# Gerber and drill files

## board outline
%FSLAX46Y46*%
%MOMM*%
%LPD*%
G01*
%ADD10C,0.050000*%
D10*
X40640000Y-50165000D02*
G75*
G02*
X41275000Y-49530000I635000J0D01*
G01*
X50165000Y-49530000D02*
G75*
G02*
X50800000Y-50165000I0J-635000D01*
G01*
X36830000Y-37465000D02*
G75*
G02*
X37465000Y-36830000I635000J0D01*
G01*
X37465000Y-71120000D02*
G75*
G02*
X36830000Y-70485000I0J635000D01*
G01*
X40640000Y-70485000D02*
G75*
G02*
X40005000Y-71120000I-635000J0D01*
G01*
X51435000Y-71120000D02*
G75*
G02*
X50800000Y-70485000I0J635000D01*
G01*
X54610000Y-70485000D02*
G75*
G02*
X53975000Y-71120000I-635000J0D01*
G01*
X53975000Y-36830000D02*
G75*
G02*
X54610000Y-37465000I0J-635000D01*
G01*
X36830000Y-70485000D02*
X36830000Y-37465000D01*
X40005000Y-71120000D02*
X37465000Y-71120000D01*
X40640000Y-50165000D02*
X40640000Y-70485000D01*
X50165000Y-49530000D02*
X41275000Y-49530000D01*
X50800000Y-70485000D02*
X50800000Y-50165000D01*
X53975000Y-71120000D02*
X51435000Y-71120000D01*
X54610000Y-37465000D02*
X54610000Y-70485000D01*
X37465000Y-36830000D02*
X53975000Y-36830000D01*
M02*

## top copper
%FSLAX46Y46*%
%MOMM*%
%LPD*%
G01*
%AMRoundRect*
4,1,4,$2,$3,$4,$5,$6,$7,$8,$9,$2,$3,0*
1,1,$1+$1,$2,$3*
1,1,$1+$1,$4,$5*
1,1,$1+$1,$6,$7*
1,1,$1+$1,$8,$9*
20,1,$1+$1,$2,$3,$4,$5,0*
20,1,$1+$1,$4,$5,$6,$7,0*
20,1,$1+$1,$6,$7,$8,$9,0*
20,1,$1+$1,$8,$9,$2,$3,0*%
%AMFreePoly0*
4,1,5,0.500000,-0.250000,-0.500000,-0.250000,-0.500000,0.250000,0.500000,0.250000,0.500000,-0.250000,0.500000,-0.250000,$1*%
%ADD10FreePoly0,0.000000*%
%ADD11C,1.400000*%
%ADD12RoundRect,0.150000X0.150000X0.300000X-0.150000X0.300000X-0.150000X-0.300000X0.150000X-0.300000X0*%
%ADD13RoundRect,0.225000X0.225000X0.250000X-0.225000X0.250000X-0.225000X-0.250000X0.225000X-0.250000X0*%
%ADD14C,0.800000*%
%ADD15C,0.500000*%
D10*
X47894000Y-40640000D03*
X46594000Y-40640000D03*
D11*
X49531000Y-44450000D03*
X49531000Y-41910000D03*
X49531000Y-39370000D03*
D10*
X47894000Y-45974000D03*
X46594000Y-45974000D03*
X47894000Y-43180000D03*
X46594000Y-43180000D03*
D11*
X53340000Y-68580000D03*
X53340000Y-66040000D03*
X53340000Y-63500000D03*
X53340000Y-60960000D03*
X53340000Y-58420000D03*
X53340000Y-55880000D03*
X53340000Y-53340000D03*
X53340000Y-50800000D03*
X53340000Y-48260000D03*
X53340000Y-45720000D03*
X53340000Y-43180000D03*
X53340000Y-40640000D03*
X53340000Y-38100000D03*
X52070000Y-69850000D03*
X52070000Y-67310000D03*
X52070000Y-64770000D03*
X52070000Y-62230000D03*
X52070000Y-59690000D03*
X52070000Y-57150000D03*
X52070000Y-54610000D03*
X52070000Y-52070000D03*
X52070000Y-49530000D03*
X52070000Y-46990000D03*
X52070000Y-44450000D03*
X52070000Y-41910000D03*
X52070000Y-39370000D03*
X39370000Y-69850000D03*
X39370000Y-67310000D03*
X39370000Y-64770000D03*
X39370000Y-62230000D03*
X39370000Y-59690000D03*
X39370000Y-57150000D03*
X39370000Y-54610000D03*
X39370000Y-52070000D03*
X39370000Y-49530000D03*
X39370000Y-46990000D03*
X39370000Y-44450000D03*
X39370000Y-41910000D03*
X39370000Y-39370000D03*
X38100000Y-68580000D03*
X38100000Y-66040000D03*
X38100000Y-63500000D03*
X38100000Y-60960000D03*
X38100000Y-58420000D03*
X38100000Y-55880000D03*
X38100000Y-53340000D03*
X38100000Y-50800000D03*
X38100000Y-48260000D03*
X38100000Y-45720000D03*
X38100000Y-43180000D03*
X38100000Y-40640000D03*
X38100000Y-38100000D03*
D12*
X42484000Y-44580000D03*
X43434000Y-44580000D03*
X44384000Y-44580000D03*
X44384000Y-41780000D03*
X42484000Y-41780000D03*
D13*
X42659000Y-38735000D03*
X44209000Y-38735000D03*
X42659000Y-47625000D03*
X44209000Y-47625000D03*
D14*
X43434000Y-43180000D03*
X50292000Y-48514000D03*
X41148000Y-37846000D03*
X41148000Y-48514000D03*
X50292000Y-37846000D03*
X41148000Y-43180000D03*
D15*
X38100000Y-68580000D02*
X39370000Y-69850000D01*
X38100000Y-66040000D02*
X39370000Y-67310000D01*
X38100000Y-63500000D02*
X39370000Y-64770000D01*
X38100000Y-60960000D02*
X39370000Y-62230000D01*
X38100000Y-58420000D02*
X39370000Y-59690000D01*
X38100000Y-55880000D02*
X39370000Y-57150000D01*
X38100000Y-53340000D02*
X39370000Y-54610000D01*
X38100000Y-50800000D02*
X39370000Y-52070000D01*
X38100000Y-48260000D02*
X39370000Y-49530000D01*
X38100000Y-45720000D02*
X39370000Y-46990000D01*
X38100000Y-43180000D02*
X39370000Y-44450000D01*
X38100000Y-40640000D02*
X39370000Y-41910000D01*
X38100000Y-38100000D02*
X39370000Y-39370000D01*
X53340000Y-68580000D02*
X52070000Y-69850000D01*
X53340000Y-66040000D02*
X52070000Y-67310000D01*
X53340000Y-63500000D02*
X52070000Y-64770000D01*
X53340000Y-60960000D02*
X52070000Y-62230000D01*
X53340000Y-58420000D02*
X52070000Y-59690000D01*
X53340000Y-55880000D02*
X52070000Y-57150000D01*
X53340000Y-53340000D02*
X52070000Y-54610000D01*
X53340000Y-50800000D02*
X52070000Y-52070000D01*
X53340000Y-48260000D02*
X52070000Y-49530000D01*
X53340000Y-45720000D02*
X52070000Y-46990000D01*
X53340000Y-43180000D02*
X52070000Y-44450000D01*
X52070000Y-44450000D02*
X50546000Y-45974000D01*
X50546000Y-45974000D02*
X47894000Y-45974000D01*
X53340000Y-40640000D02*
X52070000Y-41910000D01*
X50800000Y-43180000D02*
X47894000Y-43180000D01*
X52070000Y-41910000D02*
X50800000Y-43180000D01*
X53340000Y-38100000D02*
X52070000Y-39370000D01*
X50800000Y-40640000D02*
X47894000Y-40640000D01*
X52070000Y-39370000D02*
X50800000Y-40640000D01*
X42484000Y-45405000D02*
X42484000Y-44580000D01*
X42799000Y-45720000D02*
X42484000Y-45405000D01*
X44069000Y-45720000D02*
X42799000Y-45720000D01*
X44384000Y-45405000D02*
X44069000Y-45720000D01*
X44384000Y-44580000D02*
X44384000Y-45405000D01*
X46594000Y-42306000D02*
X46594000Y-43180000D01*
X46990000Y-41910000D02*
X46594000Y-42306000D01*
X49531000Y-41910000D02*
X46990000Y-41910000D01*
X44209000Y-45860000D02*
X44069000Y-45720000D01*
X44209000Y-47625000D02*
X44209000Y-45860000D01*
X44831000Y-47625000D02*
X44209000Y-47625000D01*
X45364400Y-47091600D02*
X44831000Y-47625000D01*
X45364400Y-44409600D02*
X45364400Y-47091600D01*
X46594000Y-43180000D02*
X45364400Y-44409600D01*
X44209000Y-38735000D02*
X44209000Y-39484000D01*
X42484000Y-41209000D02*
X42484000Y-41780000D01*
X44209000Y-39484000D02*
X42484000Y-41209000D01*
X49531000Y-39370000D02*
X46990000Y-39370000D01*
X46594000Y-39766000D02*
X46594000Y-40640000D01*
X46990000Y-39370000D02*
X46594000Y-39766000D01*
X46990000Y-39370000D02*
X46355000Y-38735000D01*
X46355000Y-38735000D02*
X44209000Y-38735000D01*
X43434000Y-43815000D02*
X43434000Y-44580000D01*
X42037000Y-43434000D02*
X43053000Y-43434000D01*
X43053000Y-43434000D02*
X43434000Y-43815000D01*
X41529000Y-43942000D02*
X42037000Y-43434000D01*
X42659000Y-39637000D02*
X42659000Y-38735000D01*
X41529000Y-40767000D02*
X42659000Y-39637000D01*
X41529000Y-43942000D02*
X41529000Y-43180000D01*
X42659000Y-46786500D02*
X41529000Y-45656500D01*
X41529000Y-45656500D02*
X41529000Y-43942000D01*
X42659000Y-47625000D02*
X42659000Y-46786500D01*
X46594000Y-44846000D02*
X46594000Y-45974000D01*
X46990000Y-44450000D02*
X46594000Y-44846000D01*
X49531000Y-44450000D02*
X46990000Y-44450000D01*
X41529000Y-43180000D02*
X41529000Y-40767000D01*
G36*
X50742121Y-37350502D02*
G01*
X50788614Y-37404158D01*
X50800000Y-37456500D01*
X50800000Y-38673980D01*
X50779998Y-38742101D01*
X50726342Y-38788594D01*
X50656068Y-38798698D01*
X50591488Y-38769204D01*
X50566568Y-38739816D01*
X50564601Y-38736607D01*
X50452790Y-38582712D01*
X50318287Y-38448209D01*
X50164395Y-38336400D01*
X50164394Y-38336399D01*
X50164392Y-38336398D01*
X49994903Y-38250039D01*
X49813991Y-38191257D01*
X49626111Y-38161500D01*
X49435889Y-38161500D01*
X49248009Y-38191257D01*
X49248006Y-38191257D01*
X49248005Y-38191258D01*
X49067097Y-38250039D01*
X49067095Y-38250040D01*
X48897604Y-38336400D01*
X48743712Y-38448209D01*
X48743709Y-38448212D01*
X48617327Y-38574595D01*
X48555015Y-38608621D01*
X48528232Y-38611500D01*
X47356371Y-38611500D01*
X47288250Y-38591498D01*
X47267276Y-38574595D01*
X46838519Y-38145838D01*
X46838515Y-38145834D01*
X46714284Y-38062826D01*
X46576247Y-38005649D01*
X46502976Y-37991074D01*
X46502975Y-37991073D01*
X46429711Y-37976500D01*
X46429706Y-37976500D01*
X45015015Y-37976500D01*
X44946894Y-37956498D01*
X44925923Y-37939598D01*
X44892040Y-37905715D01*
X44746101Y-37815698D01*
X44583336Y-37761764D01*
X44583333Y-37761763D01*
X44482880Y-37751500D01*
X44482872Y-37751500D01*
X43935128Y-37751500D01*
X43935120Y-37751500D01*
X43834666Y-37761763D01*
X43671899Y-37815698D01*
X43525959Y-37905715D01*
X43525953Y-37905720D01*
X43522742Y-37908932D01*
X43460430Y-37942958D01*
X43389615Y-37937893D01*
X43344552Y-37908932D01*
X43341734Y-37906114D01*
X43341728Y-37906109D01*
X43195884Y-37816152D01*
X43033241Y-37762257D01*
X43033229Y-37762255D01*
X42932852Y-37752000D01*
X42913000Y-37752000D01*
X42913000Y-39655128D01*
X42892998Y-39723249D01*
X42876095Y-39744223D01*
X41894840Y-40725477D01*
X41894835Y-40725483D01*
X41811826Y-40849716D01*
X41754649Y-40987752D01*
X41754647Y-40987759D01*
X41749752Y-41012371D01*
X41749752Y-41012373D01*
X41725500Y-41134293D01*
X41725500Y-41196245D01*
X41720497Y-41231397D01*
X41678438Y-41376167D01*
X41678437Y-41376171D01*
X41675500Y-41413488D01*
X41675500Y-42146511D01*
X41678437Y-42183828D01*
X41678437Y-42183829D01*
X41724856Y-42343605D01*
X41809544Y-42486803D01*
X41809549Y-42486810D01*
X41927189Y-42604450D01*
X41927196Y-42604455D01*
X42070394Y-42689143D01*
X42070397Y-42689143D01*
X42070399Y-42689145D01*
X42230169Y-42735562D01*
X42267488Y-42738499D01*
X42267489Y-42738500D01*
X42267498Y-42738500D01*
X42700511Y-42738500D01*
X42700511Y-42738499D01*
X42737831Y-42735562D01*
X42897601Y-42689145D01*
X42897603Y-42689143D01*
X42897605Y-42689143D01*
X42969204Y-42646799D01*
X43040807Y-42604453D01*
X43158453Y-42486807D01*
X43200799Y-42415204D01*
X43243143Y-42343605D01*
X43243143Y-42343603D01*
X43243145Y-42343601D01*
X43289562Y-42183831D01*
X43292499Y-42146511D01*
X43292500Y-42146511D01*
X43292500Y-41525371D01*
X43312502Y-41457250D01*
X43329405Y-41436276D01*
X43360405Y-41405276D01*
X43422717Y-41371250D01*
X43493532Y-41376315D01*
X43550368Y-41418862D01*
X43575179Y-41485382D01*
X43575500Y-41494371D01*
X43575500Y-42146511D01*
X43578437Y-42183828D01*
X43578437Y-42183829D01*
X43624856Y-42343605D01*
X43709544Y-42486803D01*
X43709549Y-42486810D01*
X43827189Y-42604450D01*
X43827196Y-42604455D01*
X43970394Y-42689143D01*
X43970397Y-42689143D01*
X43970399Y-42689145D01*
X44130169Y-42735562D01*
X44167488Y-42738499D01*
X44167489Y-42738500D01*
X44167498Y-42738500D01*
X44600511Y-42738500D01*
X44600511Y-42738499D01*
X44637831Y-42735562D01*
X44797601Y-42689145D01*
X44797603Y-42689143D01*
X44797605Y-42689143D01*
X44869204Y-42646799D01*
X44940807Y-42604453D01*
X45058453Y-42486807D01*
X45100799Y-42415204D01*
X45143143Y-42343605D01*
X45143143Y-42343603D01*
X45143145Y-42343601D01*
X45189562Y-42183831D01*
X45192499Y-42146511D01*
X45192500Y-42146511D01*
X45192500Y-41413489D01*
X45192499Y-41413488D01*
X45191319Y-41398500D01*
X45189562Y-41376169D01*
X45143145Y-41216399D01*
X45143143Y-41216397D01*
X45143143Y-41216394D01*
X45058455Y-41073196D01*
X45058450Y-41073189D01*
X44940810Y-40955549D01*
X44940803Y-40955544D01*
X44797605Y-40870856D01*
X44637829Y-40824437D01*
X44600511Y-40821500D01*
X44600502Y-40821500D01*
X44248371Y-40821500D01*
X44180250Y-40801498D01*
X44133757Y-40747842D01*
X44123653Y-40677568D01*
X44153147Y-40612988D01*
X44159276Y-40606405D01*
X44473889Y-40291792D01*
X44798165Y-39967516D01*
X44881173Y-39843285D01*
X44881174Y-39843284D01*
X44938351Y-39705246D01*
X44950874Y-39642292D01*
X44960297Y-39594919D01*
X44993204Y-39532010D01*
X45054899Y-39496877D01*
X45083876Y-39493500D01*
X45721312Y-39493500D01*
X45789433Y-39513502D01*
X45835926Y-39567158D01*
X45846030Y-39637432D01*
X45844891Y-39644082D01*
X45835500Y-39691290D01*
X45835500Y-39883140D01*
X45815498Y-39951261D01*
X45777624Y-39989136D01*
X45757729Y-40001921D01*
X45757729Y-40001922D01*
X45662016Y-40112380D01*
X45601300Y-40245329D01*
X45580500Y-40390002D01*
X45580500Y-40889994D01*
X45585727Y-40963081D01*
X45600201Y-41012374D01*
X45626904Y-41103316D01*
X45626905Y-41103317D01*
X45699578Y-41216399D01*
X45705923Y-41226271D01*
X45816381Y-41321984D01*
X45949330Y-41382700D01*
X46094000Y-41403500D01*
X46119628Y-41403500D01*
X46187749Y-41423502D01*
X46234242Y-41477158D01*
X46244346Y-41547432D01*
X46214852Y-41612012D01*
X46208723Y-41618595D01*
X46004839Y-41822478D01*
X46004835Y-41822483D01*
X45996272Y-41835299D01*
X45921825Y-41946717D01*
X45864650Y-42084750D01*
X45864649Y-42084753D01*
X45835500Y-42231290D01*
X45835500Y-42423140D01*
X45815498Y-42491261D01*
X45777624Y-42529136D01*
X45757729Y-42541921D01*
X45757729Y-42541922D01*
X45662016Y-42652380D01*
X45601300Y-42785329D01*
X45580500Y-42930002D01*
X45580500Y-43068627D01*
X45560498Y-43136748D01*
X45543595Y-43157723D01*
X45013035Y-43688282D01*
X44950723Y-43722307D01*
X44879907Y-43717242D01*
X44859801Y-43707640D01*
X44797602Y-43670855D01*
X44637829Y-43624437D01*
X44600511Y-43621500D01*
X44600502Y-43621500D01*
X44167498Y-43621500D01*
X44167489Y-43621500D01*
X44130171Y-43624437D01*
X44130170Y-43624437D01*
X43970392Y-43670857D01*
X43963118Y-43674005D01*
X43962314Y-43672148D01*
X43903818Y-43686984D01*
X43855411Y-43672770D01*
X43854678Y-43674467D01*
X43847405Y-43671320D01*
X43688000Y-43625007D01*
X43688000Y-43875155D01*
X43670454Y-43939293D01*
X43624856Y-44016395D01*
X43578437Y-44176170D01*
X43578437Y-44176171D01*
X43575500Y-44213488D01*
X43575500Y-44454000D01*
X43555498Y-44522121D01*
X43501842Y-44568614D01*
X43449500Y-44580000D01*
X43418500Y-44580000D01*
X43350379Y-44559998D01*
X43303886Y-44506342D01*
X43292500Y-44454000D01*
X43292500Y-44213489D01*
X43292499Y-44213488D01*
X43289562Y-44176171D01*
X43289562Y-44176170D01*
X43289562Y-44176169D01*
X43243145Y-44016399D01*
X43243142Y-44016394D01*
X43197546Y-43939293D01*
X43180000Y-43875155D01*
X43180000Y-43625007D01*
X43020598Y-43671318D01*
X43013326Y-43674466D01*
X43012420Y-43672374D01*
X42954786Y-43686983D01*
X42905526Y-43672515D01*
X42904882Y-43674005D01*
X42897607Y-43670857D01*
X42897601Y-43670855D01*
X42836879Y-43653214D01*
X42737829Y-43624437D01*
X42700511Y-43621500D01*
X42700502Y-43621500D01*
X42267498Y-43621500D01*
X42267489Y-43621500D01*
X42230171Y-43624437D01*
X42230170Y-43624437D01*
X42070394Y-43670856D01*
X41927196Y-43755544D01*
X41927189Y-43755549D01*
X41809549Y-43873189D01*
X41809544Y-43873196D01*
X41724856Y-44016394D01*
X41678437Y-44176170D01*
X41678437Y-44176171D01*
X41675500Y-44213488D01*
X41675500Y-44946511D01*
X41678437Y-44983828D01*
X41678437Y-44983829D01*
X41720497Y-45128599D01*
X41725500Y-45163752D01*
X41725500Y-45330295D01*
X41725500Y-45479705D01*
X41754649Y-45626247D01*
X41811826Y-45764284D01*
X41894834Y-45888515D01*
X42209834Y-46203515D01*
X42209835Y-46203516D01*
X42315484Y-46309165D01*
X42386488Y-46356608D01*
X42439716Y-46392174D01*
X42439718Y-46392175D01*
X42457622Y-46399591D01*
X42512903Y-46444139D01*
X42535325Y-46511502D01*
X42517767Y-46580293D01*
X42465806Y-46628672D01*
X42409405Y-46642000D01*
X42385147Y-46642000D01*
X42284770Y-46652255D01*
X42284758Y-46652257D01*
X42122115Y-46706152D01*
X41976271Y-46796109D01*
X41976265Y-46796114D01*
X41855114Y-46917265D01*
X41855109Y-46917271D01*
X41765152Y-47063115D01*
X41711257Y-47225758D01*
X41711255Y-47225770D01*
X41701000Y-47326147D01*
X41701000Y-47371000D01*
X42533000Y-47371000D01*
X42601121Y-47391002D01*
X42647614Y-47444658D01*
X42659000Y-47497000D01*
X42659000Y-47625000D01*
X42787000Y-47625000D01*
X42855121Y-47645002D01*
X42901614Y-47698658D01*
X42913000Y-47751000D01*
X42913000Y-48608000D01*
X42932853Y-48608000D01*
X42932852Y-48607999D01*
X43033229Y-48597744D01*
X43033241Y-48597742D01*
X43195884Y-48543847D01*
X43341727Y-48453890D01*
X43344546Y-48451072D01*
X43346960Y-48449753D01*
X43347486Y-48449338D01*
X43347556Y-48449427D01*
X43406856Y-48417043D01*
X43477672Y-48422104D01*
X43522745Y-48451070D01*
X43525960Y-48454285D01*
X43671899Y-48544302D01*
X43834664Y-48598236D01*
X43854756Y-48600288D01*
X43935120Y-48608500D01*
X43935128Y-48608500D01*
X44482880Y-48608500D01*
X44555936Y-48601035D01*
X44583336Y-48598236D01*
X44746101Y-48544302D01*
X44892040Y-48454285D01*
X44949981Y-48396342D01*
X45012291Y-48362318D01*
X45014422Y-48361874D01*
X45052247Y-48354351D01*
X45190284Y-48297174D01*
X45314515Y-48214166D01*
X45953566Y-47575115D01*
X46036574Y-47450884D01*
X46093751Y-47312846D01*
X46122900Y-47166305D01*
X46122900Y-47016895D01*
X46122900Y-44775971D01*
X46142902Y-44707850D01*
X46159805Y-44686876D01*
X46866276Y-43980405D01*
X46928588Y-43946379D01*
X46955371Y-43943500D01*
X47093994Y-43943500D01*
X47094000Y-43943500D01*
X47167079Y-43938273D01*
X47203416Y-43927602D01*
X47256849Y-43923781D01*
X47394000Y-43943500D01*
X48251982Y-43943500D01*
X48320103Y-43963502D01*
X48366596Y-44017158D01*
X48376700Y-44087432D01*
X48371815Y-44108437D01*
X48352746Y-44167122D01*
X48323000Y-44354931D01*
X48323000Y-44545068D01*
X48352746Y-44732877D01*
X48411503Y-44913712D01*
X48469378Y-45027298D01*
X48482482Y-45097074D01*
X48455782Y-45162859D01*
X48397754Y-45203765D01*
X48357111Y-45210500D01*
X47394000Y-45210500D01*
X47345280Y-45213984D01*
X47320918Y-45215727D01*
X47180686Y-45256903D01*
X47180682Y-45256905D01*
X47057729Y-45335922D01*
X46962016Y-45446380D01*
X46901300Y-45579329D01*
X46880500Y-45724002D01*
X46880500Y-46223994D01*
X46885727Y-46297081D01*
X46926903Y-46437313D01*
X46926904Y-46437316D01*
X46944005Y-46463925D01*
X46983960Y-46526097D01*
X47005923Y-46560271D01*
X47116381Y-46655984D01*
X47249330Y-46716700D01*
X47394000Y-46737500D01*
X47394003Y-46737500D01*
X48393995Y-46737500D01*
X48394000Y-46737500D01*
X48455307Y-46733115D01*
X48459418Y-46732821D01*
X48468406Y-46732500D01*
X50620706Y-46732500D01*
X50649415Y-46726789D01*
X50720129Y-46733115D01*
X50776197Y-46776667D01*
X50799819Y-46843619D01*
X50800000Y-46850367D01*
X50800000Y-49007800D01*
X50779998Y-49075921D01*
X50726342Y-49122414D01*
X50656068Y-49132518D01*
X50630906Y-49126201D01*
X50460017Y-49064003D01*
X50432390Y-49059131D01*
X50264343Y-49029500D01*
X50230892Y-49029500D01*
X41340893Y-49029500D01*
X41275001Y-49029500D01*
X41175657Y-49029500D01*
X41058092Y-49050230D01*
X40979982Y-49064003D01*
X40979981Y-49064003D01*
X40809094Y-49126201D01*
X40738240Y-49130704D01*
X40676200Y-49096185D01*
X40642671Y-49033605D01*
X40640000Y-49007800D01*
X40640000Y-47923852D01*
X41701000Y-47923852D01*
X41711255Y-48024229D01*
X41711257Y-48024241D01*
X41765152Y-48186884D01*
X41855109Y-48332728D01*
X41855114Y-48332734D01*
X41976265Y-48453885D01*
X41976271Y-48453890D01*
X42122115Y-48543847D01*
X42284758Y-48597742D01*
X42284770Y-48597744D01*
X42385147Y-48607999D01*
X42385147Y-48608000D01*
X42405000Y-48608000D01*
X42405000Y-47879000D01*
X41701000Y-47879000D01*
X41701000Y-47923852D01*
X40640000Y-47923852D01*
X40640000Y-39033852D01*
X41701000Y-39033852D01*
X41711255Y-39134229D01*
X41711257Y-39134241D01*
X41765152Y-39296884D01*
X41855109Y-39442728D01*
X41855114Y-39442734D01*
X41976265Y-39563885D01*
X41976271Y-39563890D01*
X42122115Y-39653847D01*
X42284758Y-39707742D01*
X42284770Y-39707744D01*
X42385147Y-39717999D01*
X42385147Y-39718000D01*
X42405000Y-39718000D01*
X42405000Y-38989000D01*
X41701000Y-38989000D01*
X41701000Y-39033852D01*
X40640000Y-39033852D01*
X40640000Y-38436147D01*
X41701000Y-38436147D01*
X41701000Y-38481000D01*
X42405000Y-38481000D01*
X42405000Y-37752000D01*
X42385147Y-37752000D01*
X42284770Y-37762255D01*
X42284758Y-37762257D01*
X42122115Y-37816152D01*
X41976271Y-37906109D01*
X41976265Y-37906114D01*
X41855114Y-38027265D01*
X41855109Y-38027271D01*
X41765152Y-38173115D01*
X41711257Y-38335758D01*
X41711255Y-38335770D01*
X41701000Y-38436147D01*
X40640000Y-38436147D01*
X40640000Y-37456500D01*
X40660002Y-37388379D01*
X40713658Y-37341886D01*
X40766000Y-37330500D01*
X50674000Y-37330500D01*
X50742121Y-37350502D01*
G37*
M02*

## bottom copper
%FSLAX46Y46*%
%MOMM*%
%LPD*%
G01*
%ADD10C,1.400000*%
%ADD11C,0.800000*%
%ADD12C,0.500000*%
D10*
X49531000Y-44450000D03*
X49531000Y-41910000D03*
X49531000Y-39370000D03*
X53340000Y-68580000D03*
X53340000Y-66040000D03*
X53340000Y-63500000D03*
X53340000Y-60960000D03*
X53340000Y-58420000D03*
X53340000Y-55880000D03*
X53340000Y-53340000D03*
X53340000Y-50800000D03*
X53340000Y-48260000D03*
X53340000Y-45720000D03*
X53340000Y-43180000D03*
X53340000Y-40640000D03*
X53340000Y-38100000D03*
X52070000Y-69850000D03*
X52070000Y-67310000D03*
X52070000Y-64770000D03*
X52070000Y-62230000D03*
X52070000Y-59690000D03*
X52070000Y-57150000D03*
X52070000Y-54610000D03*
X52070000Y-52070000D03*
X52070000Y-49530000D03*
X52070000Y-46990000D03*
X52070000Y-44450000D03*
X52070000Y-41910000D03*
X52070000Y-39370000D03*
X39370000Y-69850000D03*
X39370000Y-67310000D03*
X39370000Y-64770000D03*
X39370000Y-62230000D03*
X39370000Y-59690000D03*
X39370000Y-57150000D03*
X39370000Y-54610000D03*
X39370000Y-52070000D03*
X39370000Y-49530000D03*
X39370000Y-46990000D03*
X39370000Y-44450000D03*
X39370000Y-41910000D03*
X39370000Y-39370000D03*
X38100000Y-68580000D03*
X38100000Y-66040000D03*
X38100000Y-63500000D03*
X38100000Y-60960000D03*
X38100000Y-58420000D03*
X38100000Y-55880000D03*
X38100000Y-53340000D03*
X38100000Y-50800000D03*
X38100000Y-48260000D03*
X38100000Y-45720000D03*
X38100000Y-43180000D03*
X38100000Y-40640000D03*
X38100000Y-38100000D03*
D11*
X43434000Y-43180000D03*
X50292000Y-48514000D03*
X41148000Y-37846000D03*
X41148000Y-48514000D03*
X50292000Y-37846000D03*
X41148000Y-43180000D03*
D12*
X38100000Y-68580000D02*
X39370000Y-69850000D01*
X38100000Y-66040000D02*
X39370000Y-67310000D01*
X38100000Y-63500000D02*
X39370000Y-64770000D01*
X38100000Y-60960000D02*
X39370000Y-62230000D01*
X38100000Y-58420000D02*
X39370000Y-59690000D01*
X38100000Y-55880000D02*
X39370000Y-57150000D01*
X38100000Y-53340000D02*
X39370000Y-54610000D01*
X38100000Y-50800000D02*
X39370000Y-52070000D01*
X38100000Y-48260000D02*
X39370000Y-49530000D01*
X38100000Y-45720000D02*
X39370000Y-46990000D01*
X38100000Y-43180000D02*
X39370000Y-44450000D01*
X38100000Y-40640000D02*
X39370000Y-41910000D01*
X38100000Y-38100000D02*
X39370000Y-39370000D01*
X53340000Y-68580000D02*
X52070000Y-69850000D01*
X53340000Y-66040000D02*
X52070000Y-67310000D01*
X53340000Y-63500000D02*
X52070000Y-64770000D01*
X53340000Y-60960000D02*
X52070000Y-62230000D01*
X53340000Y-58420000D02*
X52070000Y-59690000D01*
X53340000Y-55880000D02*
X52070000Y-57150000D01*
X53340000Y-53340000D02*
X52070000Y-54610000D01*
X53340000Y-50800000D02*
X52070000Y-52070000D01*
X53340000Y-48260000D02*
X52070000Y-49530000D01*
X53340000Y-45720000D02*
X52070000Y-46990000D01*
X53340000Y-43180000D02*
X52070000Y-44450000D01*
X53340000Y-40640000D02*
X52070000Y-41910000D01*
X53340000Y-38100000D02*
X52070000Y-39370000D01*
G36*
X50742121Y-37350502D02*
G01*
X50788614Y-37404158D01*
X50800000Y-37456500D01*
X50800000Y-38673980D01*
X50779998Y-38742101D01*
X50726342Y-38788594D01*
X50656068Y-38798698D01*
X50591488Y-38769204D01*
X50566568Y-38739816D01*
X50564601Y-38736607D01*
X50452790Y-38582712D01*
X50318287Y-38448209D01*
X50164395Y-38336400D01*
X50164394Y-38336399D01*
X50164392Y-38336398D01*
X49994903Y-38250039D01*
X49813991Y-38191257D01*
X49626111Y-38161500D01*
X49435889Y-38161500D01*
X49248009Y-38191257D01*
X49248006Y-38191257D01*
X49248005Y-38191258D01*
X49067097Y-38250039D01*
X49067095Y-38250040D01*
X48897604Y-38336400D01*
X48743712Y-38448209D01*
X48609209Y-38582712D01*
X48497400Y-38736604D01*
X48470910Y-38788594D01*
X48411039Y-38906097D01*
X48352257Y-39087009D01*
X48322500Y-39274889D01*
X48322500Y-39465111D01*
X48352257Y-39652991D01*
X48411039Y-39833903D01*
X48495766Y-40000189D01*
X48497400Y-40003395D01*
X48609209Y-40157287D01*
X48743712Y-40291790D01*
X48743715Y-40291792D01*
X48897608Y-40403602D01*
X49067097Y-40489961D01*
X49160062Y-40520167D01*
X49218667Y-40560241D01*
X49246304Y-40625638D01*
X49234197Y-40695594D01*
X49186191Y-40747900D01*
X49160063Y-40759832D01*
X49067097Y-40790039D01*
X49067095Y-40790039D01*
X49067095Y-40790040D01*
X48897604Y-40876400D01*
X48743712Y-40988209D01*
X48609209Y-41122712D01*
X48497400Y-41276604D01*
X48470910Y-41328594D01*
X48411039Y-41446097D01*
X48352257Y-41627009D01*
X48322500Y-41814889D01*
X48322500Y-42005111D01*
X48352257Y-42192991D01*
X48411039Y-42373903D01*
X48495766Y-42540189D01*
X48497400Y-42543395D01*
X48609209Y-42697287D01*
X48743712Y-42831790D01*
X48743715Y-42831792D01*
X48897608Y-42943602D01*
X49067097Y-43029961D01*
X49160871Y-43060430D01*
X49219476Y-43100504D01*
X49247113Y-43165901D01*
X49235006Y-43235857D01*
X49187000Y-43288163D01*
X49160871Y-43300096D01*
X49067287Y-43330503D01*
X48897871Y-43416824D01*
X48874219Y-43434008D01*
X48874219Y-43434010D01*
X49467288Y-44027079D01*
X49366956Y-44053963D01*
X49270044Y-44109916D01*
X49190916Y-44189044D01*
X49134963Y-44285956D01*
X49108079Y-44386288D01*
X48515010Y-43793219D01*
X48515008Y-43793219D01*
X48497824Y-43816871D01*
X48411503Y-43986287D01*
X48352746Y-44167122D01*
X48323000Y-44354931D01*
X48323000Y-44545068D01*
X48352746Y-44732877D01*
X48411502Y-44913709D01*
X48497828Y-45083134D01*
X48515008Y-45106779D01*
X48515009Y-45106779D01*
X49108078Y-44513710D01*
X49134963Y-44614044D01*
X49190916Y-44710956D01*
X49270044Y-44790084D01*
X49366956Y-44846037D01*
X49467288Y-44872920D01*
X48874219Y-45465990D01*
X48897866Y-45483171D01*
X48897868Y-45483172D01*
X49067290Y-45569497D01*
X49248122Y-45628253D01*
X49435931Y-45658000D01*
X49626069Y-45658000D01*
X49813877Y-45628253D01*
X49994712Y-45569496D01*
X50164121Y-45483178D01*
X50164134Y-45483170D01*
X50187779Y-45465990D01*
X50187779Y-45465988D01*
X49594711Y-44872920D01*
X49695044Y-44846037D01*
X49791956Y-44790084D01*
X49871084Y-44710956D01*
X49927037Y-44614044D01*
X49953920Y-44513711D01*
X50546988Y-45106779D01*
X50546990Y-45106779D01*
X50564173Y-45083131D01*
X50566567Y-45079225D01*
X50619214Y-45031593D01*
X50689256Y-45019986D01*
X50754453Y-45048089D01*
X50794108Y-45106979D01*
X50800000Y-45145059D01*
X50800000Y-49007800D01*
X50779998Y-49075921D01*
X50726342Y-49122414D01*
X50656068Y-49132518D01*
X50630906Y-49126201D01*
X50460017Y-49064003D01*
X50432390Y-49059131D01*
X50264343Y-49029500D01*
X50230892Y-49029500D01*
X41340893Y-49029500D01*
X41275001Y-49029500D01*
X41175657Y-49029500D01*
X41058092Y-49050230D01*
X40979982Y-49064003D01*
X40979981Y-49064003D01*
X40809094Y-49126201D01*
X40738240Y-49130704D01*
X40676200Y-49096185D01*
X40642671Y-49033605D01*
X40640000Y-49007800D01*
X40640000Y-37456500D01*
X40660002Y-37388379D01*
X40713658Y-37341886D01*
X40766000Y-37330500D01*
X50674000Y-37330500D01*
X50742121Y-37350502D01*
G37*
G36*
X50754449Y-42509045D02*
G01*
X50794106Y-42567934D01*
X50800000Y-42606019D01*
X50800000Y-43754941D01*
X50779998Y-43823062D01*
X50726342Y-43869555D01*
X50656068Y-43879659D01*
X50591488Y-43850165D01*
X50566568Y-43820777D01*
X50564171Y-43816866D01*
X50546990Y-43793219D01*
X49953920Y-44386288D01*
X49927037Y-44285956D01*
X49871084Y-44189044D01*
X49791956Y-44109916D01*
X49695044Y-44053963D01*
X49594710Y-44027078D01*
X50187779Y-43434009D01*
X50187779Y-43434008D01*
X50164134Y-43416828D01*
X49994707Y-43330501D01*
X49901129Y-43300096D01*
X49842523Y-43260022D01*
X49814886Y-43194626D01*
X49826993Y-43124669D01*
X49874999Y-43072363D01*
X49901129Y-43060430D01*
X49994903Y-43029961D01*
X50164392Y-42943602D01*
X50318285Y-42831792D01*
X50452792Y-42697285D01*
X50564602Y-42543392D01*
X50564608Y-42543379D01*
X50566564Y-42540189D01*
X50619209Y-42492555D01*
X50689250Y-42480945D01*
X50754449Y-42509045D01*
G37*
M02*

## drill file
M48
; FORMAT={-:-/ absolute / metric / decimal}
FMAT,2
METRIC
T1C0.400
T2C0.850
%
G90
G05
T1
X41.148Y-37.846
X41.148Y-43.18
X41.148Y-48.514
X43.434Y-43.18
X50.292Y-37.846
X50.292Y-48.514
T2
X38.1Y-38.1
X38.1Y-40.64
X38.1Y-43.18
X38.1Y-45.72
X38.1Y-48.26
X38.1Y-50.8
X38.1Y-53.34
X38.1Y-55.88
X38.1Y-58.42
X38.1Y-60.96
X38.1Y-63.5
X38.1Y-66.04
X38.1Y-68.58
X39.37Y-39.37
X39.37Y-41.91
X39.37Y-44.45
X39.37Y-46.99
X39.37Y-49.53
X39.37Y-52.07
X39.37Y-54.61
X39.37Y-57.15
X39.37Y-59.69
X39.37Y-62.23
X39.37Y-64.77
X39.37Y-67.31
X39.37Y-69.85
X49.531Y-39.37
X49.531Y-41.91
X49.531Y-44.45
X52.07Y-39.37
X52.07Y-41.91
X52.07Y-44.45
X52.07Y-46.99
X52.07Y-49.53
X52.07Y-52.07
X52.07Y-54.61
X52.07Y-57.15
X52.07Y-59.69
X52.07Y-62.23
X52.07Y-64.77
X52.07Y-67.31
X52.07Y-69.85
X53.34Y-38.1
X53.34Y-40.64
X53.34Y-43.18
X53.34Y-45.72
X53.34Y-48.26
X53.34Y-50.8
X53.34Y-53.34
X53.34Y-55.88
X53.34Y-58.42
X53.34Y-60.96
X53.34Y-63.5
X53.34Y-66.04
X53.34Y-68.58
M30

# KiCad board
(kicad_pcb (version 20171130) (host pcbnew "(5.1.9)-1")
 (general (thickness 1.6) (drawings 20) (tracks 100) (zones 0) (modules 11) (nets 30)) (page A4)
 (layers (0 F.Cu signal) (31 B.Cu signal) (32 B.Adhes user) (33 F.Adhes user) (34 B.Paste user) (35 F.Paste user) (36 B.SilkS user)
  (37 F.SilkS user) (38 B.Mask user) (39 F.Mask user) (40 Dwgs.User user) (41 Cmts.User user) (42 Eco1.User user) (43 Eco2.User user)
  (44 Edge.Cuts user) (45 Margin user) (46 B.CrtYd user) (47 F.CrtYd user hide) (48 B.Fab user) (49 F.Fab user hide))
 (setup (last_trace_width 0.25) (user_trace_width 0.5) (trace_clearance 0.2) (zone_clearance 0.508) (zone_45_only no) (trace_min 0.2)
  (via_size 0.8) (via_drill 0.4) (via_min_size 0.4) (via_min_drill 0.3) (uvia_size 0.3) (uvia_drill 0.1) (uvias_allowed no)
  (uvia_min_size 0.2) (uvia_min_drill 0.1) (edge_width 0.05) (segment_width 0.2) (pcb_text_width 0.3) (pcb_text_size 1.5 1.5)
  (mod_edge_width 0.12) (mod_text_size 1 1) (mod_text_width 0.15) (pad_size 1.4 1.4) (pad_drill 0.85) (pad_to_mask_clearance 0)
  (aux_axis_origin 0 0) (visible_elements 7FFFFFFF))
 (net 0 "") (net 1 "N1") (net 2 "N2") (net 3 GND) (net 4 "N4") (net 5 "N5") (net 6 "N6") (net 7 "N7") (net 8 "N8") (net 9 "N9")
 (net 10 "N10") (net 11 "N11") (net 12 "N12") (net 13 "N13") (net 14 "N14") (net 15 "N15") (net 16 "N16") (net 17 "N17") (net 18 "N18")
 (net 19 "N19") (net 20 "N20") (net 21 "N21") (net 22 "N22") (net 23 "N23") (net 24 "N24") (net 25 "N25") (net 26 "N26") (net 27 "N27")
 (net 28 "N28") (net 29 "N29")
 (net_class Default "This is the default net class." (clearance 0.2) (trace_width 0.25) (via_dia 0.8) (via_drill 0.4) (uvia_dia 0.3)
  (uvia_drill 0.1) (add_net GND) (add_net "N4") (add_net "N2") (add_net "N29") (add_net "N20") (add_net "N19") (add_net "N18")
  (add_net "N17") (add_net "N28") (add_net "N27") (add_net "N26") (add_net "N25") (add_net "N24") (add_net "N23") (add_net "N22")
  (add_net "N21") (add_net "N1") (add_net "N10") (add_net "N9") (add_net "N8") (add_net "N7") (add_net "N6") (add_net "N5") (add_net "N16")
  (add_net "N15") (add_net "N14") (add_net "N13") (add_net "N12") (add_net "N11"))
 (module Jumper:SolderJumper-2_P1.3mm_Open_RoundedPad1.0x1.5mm (layer F.Cu) (at 47.244 40.64)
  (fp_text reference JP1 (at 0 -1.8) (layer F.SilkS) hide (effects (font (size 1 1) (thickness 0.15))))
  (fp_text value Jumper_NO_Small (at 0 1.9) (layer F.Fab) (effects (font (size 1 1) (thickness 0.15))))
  (pad 2 smd custom (at 0.65 0) (size 1 0.5) (layers F.Cu F.Mask) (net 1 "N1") (zone_connect 2) (options (clearance outline) (anchor rect))
   (primitives))
  (pad 1 smd custom (at -0.65 0) (size 1 0.5) (layers F.Cu F.Mask) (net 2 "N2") (zone_connect 2) (options (clearance outline) (anchor rect))
   (primitives)))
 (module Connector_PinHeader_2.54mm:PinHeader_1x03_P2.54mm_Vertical (layer F.Cu) (at 49.531 39.37)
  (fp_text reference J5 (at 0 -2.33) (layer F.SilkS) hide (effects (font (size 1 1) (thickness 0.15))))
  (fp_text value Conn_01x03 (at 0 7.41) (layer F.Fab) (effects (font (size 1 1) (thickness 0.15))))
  (pad 3 thru_hole circle (at 0 5.08) (size 1.4 1.4) (drill 0.85) (layers *.Cu *.Mask) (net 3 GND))
  (pad 2 thru_hole circle (at 0 2.54) (size 1.4 1.4) (drill 0.85) (layers *.Cu *.Mask) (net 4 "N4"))
  (pad 1 thru_hole circle (at 0 0) (size 1.4 1.4) (drill 0.85) (layers *.Cu *.Mask) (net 2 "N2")))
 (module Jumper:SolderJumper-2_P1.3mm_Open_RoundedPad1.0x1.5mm (layer F.Cu) (at 47.244 45.974)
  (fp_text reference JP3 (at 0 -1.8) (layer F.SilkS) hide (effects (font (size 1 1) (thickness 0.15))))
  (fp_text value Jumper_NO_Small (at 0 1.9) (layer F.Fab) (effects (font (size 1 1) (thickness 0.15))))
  (pad 2 smd custom (at 0.65 0) (size 1 0.5) (layers F.Cu F.Mask) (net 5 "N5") (zone_connect 2) (options (clearance outline) (anchor rect))
   (primitives))
  (pad 1 smd custom (at -0.65 0) (size 1 0.5) (layers F.Cu F.Mask) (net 3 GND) (zone_connect 2) (options (clearance outline) (anchor rect))
   (primitives)))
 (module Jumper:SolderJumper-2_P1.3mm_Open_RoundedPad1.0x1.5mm (layer F.Cu) (at 47.244 43.18)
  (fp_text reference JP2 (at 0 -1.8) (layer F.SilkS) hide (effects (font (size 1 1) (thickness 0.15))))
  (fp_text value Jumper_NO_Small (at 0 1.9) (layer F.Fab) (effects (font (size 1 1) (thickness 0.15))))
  (pad 2 smd custom (at 0.65 0) (size 1 0.5) (layers F.Cu F.Mask) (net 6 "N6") (zone_connect 2) (options (clearance outline) (anchor rect))
   (primitives))
  (pad 1 smd custom (at -0.65 0) (size 1 0.5) (layers F.Cu F.Mask) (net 4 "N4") (zone_connect 2) (options (clearance outline) (anchor rect))
   (primitives)))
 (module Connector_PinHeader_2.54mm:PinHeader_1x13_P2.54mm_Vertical (layer F.Cu) (at 53.34 38.1)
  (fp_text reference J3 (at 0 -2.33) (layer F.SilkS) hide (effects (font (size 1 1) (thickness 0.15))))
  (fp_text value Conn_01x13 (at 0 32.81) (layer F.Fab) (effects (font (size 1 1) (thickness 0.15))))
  (pad 13 thru_hole circle (at 0 30.48) (size 1.4 1.4) (drill 0.85) (layers *.Cu *.Mask) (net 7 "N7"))
  (pad 12 thru_hole circle (at 0 27.94) (size 1.4 1.4) (drill 0.85) (layers *.Cu *.Mask) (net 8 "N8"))
  (pad 11 thru_hole circle (at 0 25.4) (size 1.4 1.4) (drill 0.85) (layers *.Cu *.Mask) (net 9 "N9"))
  (pad 10 thru_hole circle (at 0 22.86) (size 1.4 1.4) (drill 0.85) (layers *.Cu *.Mask) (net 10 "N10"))
  (pad 9 thru_hole circle (at 0 20.32) (size 1.4 1.4) (drill 0.85) (layers *.Cu *.Mask) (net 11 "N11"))
  (pad 8 thru_hole circle (at 0 17.78) (size 1.4 1.4) (drill 0.85) (layers *.Cu *.Mask) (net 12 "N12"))
  (pad 7 thru_hole circle (at 0 15.24) (size 1.4 1.4) (drill 0.85) (layers *.Cu *.Mask) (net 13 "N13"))
  (pad 6 thru_hole circle (at 0 12.7) (size 1.4 1.4) (drill 0.85) (layers *.Cu *.Mask) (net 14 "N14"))
  (pad 5 thru_hole circle (at 0 10.16) (size 1.4 1.4) (drill 0.85) (layers *.Cu *.Mask) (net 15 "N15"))
  (pad 4 thru_hole circle (at 0 7.62) (size 1.4 1.4) (drill 0.85) (layers *.Cu *.Mask) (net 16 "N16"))
  (pad 3 thru_hole circle (at 0 5.08) (size 1.4 1.4) (drill 0.85) (layers *.Cu *.Mask) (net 5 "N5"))
  (pad 2 thru_hole circle (at 0 2.54) (size 1.4 1.4) (drill 0.85) (layers *.Cu *.Mask) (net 6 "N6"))
  (pad 1 thru_hole circle (at 0 0) (size 1.4 1.4) (drill 0.85) (layers *.Cu *.Mask) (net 1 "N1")))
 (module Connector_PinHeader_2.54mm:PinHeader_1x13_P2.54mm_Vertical (layer F.Cu) (at 52.07 39.37)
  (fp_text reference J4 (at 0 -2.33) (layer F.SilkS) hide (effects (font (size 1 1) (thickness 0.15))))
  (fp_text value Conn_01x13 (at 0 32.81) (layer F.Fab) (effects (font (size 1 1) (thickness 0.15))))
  (pad 13 thru_hole circle (at 0 30.48) (size 1.4 1.4) (drill 0.85) (layers *.Cu *.Mask) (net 7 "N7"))
  (pad 12 thru_hole circle (at 0 27.94) (size 1.4 1.4) (drill 0.85) (layers *.Cu *.Mask) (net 8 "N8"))
  (pad 11 thru_hole circle (at 0 25.4) (size 1.4 1.4) (drill 0.85) (layers *.Cu *.Mask) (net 9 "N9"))
  (pad 10 thru_hole circle (at 0 22.86) (size 1.4 1.4) (drill 0.85) (layers *.Cu *.Mask) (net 10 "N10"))
  (pad 9 thru_hole circle (at 0 20.32) (size 1.4 1.4) (drill 0.85) (layers *.Cu *.Mask) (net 11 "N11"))
  (pad 8 thru_hole circle (at 0 17.78) (size 1.4 1.4) (drill 0.85) (layers *.Cu *.Mask) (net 12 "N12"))
  (pad 7 thru_hole circle (at 0 15.24) (size 1.4 1.4) (drill 0.85) (layers *.Cu *.Mask) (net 13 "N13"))
  (pad 6 thru_hole circle (at 0 12.7) (size 1.4 1.4) (drill 0.85) (layers *.Cu *.Mask) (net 14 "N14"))
  (pad 5 thru_hole circle (at 0 10.16) (size 1.4 1.4) (drill 0.85) (layers *.Cu *.Mask) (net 15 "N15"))
  (pad 4 thru_hole circle (at 0 7.62) (size 1.4 1.4) (drill 0.85) (layers *.Cu *.Mask) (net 16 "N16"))
  (pad 3 thru_hole circle (at 0 5.08) (size 1.4 1.4) (drill 0.85) (layers *.Cu *.Mask) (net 5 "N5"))
  (pad 2 thru_hole circle (at 0 2.54) (size 1.4 1.4) (drill 0.85) (layers *.Cu *.Mask) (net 6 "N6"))
  (pad 1 thru_hole circle (at 0 0) (size 1.4 1.4) (drill 0.85) (layers *.Cu *.Mask) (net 1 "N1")))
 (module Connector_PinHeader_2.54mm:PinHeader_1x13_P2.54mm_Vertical (layer F.Cu) (at 39.37 39.37)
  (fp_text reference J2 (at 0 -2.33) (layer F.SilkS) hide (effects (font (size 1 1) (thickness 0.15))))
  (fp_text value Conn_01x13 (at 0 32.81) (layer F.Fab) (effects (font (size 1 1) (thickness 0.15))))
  (pad 13 thru_hole circle (at 0 30.48) (size 1.4 1.4) (drill 0.85) (layers *.Cu *.Mask) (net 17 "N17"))
  (pad 12 thru_hole circle (at 0 27.94) (size 1.4 1.4) (drill 0.85) (layers *.Cu *.Mask) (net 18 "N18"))
  (pad 11 thru_hole circle (at 0 25.4) (size 1.4 1.4) (drill 0.85) (layers *.Cu *.Mask) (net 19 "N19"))
  (pad 10 thru_hole circle (at 0 22.86) (size 1.4 1.4) (drill 0.85) (layers *.Cu *.Mask) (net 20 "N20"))
  (pad 9 thru_hole circle (at 0 20.32) (size 1.4 1.4) (drill 0.85) (layers *.Cu *.Mask) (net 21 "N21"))
  (pad 8 thru_hole circle (at 0 17.78) (size 1.4 1.4) (drill 0.85) (layers *.Cu *.Mask) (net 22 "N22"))
  (pad 7 thru_hole circle (at 0 15.24) (size 1.4 1.4) (drill 0.85) (layers *.Cu *.Mask) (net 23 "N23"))
  (pad 6 thru_hole circle (at 0 12.7) (size 1.4 1.4) (drill 0.85) (layers *.Cu *.Mask) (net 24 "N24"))
  (pad 5 thru_hole circle (at 0 10.16) (size 1.4 1.4) (drill 0.85) (layers *.Cu *.Mask) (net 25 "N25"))
  (pad 4 thru_hole circle (at 0 7.62) (size 1.4 1.4) (drill 0.85) (layers *.Cu *.Mask) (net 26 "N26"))
  (pad 3 thru_hole circle (at 0 5.08) (size 1.4 1.4) (drill 0.85) (layers *.Cu *.Mask) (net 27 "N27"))
  (pad 2 thru_hole circle (at 0 2.54) (size 1.4 1.4) (drill 0.85) (layers *.Cu *.Mask) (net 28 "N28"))
  (pad 1 thru_hole circle (at 0 0) (size 1.4 1.4) (drill 0.85) (layers *.Cu *.Mask) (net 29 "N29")))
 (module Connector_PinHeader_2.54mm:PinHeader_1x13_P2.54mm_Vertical (layer F.Cu) (at 38.1 38.1)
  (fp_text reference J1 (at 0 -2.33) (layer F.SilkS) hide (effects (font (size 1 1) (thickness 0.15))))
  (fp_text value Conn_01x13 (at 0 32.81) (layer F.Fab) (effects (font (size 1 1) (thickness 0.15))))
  (pad 13 thru_hole circle (at 0 30.48) (size 1.4 1.4) (drill 0.85) (layers *.Cu *.Mask) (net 17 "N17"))
  (pad 12 thru_hole circle (at 0 27.94) (size 1.4 1.4) (drill 0.85) (layers *.Cu *.Mask) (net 18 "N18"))
  (pad 11 thru_hole circle (at 0 25.4) (size 1.4 1.4) (drill 0.85) (layers *.Cu *.Mask) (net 19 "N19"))
  (pad 10 thru_hole circle (at 0 22.86) (size 1.4 1.4) (drill 0.85) (layers *.Cu *.Mask) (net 20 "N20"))
  (pad 9 thru_hole circle (at 0 20.32) (size 1.4 1.4) (drill 0.85) (layers *.Cu *.Mask) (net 21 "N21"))
  (pad 8 thru_hole circle (at 0 17.78) (size 1.4 1.4) (drill 0.85) (layers *.Cu *.Mask) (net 22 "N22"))
  (pad 7 thru_hole circle (at 0 15.24) (size 1.4 1.4) (drill 0.85) (layers *.Cu *.Mask) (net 23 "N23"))
  (pad 6 thru_hole circle (at 0 12.7) (size 1.4 1.4) (drill 0.85) (layers *.Cu *.Mask) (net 24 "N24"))
  (pad 5 thru_hole circle (at 0 10.16) (size 1.4 1.4) (drill 0.85) (layers *.Cu *.Mask) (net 25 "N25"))
  (pad 4 thru_hole circle (at 0 7.62) (size 1.4 1.4) (drill 0.85) (layers *.Cu *.Mask) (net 26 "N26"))
  (pad 3 thru_hole circle (at 0 5.08) (size 1.4 1.4) (drill 0.85) (layers *.Cu *.Mask) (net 27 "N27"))
  (pad 2 thru_hole circle (at 0 2.54) (size 1.4 1.4) (drill 0.85) (layers *.Cu *.Mask) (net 28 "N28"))
  (pad 1 thru_hole circle (at 0 0) (size 1.4 1.4) (drill 0.85) (layers *.Cu *.Mask) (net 29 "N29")))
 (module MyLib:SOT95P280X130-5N (layer F.Cu) (at 43.434 43.18 90)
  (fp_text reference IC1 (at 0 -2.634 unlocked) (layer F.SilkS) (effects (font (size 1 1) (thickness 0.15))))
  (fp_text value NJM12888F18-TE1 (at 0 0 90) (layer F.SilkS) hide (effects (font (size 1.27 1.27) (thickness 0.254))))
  (pad 1 smd roundrect (at -1.4 -0.95 180) (size 0.6 0.9) (layers F.Cu F.Paste F.Mask) (roundrect_rratio 0.25) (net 4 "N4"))
  (pad 2 smd roundrect (at -1.4 0 180) (size 0.6 0.9) (layers F.Cu F.Paste F.Mask) (roundrect_rratio 0.25) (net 3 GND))
  (pad 3 smd roundrect (at -1.4 0.95 180) (size 0.6 0.9) (layers F.Cu F.Paste F.Mask) (roundrect_rratio 0.25) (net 4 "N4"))
  (pad 4 smd roundrect (at 1.4 0.95 180) (size 0.6 0.9) (layers F.Cu F.Paste F.Mask) (roundrect_rratio 0.25))
  (pad 5 smd roundrect (at 1.4 -0.95 180) (size 0.6 0.9) (layers F.Cu F.Paste F.Mask) (roundrect_rratio 0.25) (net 2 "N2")))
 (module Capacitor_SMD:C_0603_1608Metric (layer F.Cu) (at 43.434 38.735 180)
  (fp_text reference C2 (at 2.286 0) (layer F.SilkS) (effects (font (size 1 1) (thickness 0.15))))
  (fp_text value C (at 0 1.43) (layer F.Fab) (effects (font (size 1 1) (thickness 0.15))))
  (pad 2 smd roundrect (at 0.775 0 180) (size 0.9 0.95) (layers F.Cu F.Paste F.Mask) (roundrect_rratio 0.25) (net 3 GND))
  (pad 1 smd roundrect (at -0.775 0 180) (size 0.9 0.95) (layers F.Cu F.Paste F.Mask) (roundrect_rratio 0.25) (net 2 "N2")))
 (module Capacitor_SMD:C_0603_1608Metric (layer F.Cu) (at 43.434 47.625 180)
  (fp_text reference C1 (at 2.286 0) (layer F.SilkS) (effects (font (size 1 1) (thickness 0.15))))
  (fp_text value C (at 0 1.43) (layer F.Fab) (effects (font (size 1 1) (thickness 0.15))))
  (pad 2 smd roundrect (at 0.775 0 180) (size 0.9 0.95) (layers F.Cu F.Paste F.Mask) (roundrect_rratio 0.25) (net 3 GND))
  (pad 1 smd roundrect (at -0.775 0 180) (size 0.9 0.95) (layers F.Cu F.Paste F.Mask) (roundrect_rratio 0.25) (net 4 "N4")))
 (gr_arc (start 41.275 50.165) (end 41.275 49.53) (angle -90) (layer Edge.Cuts) (width 0.05))
 (gr_arc (start 50.165 50.165) (end 50.8 50.165) (angle -90) (layer Edge.Cuts) (width 0.05))
 (gr_arc (start 37.465 37.465) (end 37.465 36.83) (angle -90) (layer Edge.Cuts) (width 0.05))
 (gr_arc (start 37.465 70.485) (end 36.83 70.485) (angle -90) (layer Edge.Cuts) (width 0.05))
 (gr_arc (start 40.005 70.485) (end 40.005 71.12) (angle -90) (layer Edge.Cuts) (width 0.05))
 (gr_arc (start 51.435 70.485) (end 50.8 70.485) (angle -90) (layer Edge.Cuts) (width 0.05))
 (gr_arc (start 53.975 70.485) (end 53.975 71.12) (angle -90) (layer Edge.Cuts) (width 0.05))
 (gr_arc (start 53.975 37.465) (end 54.61 37.465) (angle -90) (layer Edge.Cuts) (width 0.05))
 (gr_line (start 36.83 70.485) (end 36.83 37.465) (layer Edge.Cuts) (width 0.05))
 (gr_line (start 40.005 71.12) (end 37.465 71.12) (layer Edge.Cuts) (width 0.05))
 (gr_line (start 40.64 50.165) (end 40.64 70.485) (layer Edge.Cuts) (width 0.05))
 (gr_line (start 50.165 49.53) (end 41.275 49.53) (layer Edge.Cuts) (width 0.05))
 (gr_line (start 50.8 70.485) (end 50.8 50.165) (layer Edge.Cuts) (width 0.05))
 (gr_line (start 53.975 71.12) (end 51.435 71.12) (layer Edge.Cuts) (width 0.05))
 (gr_line (start 54.61 37.465) (end 54.61 70.485) (layer Edge.Cuts) (width 0.05))
 (gr_line (start 37.465 36.83) (end 53.975 36.83) (layer Edge.Cuts) (width 0.05))
 (segment (start 38.1 68.58) (end 39.37 69.85) (width 0.5) (layer B.Cu) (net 17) (status 30))
 (segment (start 38.1 68.58) (end 39.37 69.85) (width 0.5) (layer F.Cu) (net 17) (status 30))
 (segment (start 38.1 66.04) (end 39.37 67.31) (width 0.5) (layer B.Cu) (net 18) (status 30))
 (segment (start 38.1 66.04) (end 39.37 67.31) (width 0.5) (layer F.Cu) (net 18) (status 30))
 (segment (start 38.1 63.5) (end 39.37 64.77) (width 0.5) (layer B.Cu) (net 19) (status 30))
 (segment (start 38.1 63.5) (end 39.37 64.77) (width 0.5) (layer F.Cu) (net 19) (status 30))
 (segment (start 38.1 60.96) (end 39.37 62.23) (width 0.5) (layer B.Cu) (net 20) (status 30))
 (segment (start 38.1 60.96) (end 39.37 62.23) (width 0.5) (layer F.Cu) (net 20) (status 30))
 (segment (start 38.1 58.42) (end 39.37 59.69) (width 0.5) (layer B.Cu) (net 21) (status 30))
 (segment (start 38.1 58.42) (end 39.37 59.69) (width 0.5) (layer F.Cu) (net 21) (status 30))
 (segment (start 38.1 55.88) (end 39.37 57.15) (width 0.5) (layer B.Cu) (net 22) (status 30))
 (segment (start 38.1 55.88) (end 39.37 57.15) (width 0.5) (layer F.Cu) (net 22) (status 30))
 (segment (start 38.1 53.34) (end 39.37 54.61) (width 0.5) (layer B.Cu) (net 23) (status 30))
 (segment (start 38.1 53.34) (end 39.37 54.61) (width 0.5) (layer F.Cu) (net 23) (status 30))
 (segment (start 38.1 50.8) (end 39.37 52.07) (width 0.5) (layer B.Cu) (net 24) (status 30))
 (segment (start 38.1 50.8) (end 39.37 52.07) (width 0.5) (layer F.Cu) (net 24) (status 30))
 (segment (start 38.1 48.26) (end 39.37 49.53) (width 0.5) (layer B.Cu) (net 25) (status 30))
 (segment (start 38.1 48.26) (end 39.37 49.53) (width 0.5) (layer F.Cu) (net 25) (status 30))
 (segment (start 38.1 45.72) (end 39.37 46.99) (width 0.5) (layer B.Cu) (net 26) (status 30))
 (segment (start 38.1 45.72) (end 39.37 46.99) (width 0.5) (layer F.Cu) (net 26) (status 30))
 (segment (start 38.1 43.18) (end 39.37 44.45) (width 0.5) (layer B.Cu) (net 27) (status 30))
 (segment (start 38.1 43.18) (end 39.37 44.45) (width 0.5) (layer F.Cu) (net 27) (status 30))
 (segment (start 38.1 40.64) (end 39.37 41.91) (width 0.5) (layer B.Cu) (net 28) (status 30))
 (segment (start 38.1 40.64) (end 39.37 41.91) (width 0.5) (layer F.Cu) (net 28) (status 30))
 (segment (start 38.1 38.1) (end 39.37 39.37) (width 0.5) (layer B.Cu) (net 29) (status 30))
 (segment (start 38.1 38.1) (end 39.37 39.37) (width 0.5) (layer F.Cu) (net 29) (status 30))
 (segment (start 53.34 68.58) (end 52.07 69.85) (width 0.5) (layer B.Cu) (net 7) (status 30))
 (segment (start 53.34 68.58) (end 52.07 69.85) (width 0.5) (layer F.Cu) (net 7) (status 30))
 (segment (start 53.34 66.04) (end 52.07 67.31) (width 0.5) (layer B.Cu) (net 8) (status 30))
 (segment (start 53.34 66.04) (end 52.07 67.31) (width 0.5) (layer F.Cu) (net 8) (status 30))
 (segment (start 53.34 63.5) (end 52.07 64.77) (width 0.5) (layer B.Cu) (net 9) (status 30))
 (segment (start 53.34 63.5) (end 52.07 64.77) (width 0.5) (layer F.Cu) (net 9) (status 30))
 (segment (start 53.34 60.96) (end 52.07 62.23) (width 0.5) (layer B.Cu) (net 10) (status 30))
 (segment (start 53.34 60.96) (end 52.07 62.23) (width 0.5) (layer F.Cu) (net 10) (status 30))
 (segment (start 53.34 58.42) (end 52.07 59.69) (width 0.5) (layer B.Cu) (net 11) (status 30))
 (segment (start 53.34 58.42) (end 52.07 59.69) (width 0.5) (layer F.Cu) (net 11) (status 30))
 (segment (start 53.34 55.88) (end 52.07 57.15) (width 0.5) (layer B.Cu) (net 12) (status 30))
 (segment (start 53.34 55.88) (end 52.07 57.15) (width 0.5) (layer F.Cu) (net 12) (status 30))
 (segment (start 53.34 53.34) (end 52.07 54.61) (width 0.5) (layer B.Cu) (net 13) (status 30))
 (segment (start 53.34 53.34) (end 52.07 54.61) (width 0.5) (layer F.Cu) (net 13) (status 30))
 (segment (start 53.34 50.8) (end 52.07 52.07) (width 0.5) (layer B.Cu) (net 14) (status 30))
 (segment (start 53.34 50.8) (end 52.07 52.07) (width 0.5) (layer F.Cu) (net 14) (status 30))
 (segment (start 53.34 48.26) (end 52.07 49.53) (width 0.5) (layer B.Cu) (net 15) (status 30))
 (segment (start 53.34 48.26) (end 52.07 49.53) (width 0.5) (layer F.Cu) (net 15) (status 30))
 (segment (start 53.34 45.72) (end 52.07 46.99) (width 0.5) (layer B.Cu) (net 16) (status 30))
 (segment (start 53.34 45.72) (end 52.07 46.99) (width 0.5) (layer F.Cu) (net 16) (status 30))
 (segment (start 53.34 43.18) (end 52.07 44.45) (width 0.5) (layer B.Cu) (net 5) (status 30))
 (segment (start 53.34 43.18) (end 52.07 44.45) (width 0.5) (layer F.Cu) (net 5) (status 30))
 (segment (start 52.07 44.45) (end 50.546 45.974) (width 0.5) (layer F.Cu) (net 5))
 (segment (start 50.546 45.974) (end 47.894 45.974) (width 0.5) (layer F.Cu) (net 5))
 (segment (start 53.34 40.64) (end 52.07 41.91) (width 0.5) (layer B.Cu) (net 6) (status 30))
 (segment (start 53.34 40.64) (end 52.07 41.91) (width 0.5) (layer F.Cu) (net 6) (status 30))
 (segment (start 50.8 43.18) (end 47.894 43.18) (width 0.5) (layer F.Cu) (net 6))
 (segment (start 52.07 41.91) (end 50.8 43.18) (width 0.5) (layer F.Cu) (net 6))
 (segment (start 53.34 38.1) (end 52.07 39.37) (width 0.5) (layer B.Cu) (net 1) (status 30))
 (segment (start 53.34 38.1) (end 52.07 39.37) (width 0.5) (layer F.Cu) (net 1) (status 30))
 (segment (start 50.8 40.64) (end 47.894 40.64) (width 0.5) (layer F.Cu) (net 1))
 (segment (start 52.07 39.37) (end 50.8 40.64) (width 0.5) (layer F.Cu) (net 1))
 (segment (start 42.484 45.405) (end 42.484 44.58) (width 0.5) (layer F.Cu) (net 4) (status 20))
 (segment (start 42.799 45.72) (end 42.484 45.405) (width 0.5) (layer F.Cu) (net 4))
 (segment (start 44.069 45.72) (end 42.799 45.72) (width 0.5) (layer F.Cu) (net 4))
 (segment (start 44.384 45.405) (end 44.069 45.72) (width 0.5) (layer F.Cu) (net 4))
 (segment (start 44.384 44.58) (end 44.384 45.405) (width 0.5) (layer F.Cu) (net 4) (status 10))
 (segment (start 46.594 42.306) (end 46.594 43.18) (width 0.5) (layer F.Cu) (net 4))
 (segment (start 46.99 41.91) (end 46.594 42.306) (width 0.5) (layer F.Cu) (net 4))
 (segment (start 49.531 41.91) (end 46.99 41.91) (width 0.5) (layer F.Cu) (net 4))
 (segment (start 44.209 45.86) (end 44.069 45.72) (width 0.5) (layer F.Cu) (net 4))
 (segment (start 44.209 47.625) (end 44.209 45.86) (width 0.5) (layer F.Cu) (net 4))
 (segment (start 44.831 47.625) (end 44.209 47.625) (width 0.5) (layer F.Cu) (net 4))
 (segment (start 45.3644 47.0916) (end 44.831 47.625) (width 0.5) (layer F.Cu) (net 4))
 (segment (start 45.3644 44.4096) (end 45.3644 47.0916) (width 0.5) (layer F.Cu) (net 4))
 (segment (start 46.594 43.18) (end 45.3644 44.4096) (width 0.5) (layer F.Cu) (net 4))
 (segment (start 44.209 38.735) (end 44.209 39.484) (width 0.5) (layer F.Cu) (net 2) (status 10))
 (segment (start 42.484 41.209) (end 42.484 41.78) (width 0.5) (layer F.Cu) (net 2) (status 20))
 (segment (start 44.209 39.484) (end 42.484 41.209) (width 0.5) (layer F.Cu) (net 2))
 (segment (start 49.531 39.37) (end 46.99 39.37) (width 0.5) (layer F.Cu) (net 2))
 (segment (start 46.594 39.766) (end 46.594 40.64) (width 0.5) (layer F.Cu) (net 2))
 (segment (start 46.99 39.37) (end 46.594 39.766) (width 0.5) (layer F.Cu) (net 2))
 (segment (start 46.99 39.37) (end 46.355 38.735) (width 0.5) (layer F.Cu) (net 2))
 (segment (start 46.355 38.735) (end 44.209 38.735) (width 0.5) (layer F.Cu) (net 2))
 (segment (start 43.434 43.815) (end 43.434 44.58) (width 0.5) (layer F.Cu) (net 3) (status 20))
 (segment (start 42.037 43.434) (end 43.053 43.434) (width 0.5) (layer F.Cu) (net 3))
 (segment (start 43.053 43.434) (end 43.434 43.815) (width 0.5) (layer F.Cu) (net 3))
 (segment (start 41.529 43.942) (end 42.037 43.434) (width 0.5) (layer F.Cu) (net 3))
 (via (at 43.434 43.18) (size 0.8) (drill 0.4) (layers F.Cu B.Cu) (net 3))
 (segment (start 42.659 39.637) (end 42.659 38.735) (width 0.5) (layer F.Cu) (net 3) (status 20))
 (segment (start 41.529 40.767) (end 42.659 39.637) (width 0.5) (layer F.Cu) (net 3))
 (segment (start 41.529 43.942) (end 41.529 43.18) (width 0.5) (layer F.Cu) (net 3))
 (segment (start 42.659 46.7865) (end 41.529 45.6565) (width 0.5) (layer F.Cu) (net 3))
 (segment (start 41.529 45.6565) (end 41.529 43.942) (width 0.5) (layer F.Cu) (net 3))
 (segment (start 42.659 47.625) (end 42.659 46.7865) (width 0.5) (layer F.Cu) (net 3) (status 10))
 (segment (start 46.594 44.846) (end 46.594 45.974) (width 0.5) (layer F.Cu) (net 3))
 (segment (start 46.99 44.45) (end 46.594 44.846) (width 0.5) (layer F.Cu) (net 3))
 (segment (start 49.531 44.45) (end 46.99 44.45) (width 0.5) (layer F.Cu) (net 3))
 (via (at 50.292 48.514) (size 0.8) (drill 0.4) (layers F.Cu B.Cu) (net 3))
 (via (at 41.148 37.846) (size 0.8) (drill 0.4) (layers F.Cu B.Cu) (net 3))
 (via (at 41.148 48.514) (size 0.8) (drill 0.4) (layers F.Cu B.Cu) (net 3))
 (via (at 50.292 37.846) (size 0.8) (drill 0.4) (layers F.Cu B.Cu) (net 3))
 (segment (start 41.529 43.18) (end 41.529 40.767) (width 0.5) (layer F.Cu) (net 3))
 (via (at 41.148 43.18) (size 0.8) (drill 0.4) (layers F.Cu B.Cu) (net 3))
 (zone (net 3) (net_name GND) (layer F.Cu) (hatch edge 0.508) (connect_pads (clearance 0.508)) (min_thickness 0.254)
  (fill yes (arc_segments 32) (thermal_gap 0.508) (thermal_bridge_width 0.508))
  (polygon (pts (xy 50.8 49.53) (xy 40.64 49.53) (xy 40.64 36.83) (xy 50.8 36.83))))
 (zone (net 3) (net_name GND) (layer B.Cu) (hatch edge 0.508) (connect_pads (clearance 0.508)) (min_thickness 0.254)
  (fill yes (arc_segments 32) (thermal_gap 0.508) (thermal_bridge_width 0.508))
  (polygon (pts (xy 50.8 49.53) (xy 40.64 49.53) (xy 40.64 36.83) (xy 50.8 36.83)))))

